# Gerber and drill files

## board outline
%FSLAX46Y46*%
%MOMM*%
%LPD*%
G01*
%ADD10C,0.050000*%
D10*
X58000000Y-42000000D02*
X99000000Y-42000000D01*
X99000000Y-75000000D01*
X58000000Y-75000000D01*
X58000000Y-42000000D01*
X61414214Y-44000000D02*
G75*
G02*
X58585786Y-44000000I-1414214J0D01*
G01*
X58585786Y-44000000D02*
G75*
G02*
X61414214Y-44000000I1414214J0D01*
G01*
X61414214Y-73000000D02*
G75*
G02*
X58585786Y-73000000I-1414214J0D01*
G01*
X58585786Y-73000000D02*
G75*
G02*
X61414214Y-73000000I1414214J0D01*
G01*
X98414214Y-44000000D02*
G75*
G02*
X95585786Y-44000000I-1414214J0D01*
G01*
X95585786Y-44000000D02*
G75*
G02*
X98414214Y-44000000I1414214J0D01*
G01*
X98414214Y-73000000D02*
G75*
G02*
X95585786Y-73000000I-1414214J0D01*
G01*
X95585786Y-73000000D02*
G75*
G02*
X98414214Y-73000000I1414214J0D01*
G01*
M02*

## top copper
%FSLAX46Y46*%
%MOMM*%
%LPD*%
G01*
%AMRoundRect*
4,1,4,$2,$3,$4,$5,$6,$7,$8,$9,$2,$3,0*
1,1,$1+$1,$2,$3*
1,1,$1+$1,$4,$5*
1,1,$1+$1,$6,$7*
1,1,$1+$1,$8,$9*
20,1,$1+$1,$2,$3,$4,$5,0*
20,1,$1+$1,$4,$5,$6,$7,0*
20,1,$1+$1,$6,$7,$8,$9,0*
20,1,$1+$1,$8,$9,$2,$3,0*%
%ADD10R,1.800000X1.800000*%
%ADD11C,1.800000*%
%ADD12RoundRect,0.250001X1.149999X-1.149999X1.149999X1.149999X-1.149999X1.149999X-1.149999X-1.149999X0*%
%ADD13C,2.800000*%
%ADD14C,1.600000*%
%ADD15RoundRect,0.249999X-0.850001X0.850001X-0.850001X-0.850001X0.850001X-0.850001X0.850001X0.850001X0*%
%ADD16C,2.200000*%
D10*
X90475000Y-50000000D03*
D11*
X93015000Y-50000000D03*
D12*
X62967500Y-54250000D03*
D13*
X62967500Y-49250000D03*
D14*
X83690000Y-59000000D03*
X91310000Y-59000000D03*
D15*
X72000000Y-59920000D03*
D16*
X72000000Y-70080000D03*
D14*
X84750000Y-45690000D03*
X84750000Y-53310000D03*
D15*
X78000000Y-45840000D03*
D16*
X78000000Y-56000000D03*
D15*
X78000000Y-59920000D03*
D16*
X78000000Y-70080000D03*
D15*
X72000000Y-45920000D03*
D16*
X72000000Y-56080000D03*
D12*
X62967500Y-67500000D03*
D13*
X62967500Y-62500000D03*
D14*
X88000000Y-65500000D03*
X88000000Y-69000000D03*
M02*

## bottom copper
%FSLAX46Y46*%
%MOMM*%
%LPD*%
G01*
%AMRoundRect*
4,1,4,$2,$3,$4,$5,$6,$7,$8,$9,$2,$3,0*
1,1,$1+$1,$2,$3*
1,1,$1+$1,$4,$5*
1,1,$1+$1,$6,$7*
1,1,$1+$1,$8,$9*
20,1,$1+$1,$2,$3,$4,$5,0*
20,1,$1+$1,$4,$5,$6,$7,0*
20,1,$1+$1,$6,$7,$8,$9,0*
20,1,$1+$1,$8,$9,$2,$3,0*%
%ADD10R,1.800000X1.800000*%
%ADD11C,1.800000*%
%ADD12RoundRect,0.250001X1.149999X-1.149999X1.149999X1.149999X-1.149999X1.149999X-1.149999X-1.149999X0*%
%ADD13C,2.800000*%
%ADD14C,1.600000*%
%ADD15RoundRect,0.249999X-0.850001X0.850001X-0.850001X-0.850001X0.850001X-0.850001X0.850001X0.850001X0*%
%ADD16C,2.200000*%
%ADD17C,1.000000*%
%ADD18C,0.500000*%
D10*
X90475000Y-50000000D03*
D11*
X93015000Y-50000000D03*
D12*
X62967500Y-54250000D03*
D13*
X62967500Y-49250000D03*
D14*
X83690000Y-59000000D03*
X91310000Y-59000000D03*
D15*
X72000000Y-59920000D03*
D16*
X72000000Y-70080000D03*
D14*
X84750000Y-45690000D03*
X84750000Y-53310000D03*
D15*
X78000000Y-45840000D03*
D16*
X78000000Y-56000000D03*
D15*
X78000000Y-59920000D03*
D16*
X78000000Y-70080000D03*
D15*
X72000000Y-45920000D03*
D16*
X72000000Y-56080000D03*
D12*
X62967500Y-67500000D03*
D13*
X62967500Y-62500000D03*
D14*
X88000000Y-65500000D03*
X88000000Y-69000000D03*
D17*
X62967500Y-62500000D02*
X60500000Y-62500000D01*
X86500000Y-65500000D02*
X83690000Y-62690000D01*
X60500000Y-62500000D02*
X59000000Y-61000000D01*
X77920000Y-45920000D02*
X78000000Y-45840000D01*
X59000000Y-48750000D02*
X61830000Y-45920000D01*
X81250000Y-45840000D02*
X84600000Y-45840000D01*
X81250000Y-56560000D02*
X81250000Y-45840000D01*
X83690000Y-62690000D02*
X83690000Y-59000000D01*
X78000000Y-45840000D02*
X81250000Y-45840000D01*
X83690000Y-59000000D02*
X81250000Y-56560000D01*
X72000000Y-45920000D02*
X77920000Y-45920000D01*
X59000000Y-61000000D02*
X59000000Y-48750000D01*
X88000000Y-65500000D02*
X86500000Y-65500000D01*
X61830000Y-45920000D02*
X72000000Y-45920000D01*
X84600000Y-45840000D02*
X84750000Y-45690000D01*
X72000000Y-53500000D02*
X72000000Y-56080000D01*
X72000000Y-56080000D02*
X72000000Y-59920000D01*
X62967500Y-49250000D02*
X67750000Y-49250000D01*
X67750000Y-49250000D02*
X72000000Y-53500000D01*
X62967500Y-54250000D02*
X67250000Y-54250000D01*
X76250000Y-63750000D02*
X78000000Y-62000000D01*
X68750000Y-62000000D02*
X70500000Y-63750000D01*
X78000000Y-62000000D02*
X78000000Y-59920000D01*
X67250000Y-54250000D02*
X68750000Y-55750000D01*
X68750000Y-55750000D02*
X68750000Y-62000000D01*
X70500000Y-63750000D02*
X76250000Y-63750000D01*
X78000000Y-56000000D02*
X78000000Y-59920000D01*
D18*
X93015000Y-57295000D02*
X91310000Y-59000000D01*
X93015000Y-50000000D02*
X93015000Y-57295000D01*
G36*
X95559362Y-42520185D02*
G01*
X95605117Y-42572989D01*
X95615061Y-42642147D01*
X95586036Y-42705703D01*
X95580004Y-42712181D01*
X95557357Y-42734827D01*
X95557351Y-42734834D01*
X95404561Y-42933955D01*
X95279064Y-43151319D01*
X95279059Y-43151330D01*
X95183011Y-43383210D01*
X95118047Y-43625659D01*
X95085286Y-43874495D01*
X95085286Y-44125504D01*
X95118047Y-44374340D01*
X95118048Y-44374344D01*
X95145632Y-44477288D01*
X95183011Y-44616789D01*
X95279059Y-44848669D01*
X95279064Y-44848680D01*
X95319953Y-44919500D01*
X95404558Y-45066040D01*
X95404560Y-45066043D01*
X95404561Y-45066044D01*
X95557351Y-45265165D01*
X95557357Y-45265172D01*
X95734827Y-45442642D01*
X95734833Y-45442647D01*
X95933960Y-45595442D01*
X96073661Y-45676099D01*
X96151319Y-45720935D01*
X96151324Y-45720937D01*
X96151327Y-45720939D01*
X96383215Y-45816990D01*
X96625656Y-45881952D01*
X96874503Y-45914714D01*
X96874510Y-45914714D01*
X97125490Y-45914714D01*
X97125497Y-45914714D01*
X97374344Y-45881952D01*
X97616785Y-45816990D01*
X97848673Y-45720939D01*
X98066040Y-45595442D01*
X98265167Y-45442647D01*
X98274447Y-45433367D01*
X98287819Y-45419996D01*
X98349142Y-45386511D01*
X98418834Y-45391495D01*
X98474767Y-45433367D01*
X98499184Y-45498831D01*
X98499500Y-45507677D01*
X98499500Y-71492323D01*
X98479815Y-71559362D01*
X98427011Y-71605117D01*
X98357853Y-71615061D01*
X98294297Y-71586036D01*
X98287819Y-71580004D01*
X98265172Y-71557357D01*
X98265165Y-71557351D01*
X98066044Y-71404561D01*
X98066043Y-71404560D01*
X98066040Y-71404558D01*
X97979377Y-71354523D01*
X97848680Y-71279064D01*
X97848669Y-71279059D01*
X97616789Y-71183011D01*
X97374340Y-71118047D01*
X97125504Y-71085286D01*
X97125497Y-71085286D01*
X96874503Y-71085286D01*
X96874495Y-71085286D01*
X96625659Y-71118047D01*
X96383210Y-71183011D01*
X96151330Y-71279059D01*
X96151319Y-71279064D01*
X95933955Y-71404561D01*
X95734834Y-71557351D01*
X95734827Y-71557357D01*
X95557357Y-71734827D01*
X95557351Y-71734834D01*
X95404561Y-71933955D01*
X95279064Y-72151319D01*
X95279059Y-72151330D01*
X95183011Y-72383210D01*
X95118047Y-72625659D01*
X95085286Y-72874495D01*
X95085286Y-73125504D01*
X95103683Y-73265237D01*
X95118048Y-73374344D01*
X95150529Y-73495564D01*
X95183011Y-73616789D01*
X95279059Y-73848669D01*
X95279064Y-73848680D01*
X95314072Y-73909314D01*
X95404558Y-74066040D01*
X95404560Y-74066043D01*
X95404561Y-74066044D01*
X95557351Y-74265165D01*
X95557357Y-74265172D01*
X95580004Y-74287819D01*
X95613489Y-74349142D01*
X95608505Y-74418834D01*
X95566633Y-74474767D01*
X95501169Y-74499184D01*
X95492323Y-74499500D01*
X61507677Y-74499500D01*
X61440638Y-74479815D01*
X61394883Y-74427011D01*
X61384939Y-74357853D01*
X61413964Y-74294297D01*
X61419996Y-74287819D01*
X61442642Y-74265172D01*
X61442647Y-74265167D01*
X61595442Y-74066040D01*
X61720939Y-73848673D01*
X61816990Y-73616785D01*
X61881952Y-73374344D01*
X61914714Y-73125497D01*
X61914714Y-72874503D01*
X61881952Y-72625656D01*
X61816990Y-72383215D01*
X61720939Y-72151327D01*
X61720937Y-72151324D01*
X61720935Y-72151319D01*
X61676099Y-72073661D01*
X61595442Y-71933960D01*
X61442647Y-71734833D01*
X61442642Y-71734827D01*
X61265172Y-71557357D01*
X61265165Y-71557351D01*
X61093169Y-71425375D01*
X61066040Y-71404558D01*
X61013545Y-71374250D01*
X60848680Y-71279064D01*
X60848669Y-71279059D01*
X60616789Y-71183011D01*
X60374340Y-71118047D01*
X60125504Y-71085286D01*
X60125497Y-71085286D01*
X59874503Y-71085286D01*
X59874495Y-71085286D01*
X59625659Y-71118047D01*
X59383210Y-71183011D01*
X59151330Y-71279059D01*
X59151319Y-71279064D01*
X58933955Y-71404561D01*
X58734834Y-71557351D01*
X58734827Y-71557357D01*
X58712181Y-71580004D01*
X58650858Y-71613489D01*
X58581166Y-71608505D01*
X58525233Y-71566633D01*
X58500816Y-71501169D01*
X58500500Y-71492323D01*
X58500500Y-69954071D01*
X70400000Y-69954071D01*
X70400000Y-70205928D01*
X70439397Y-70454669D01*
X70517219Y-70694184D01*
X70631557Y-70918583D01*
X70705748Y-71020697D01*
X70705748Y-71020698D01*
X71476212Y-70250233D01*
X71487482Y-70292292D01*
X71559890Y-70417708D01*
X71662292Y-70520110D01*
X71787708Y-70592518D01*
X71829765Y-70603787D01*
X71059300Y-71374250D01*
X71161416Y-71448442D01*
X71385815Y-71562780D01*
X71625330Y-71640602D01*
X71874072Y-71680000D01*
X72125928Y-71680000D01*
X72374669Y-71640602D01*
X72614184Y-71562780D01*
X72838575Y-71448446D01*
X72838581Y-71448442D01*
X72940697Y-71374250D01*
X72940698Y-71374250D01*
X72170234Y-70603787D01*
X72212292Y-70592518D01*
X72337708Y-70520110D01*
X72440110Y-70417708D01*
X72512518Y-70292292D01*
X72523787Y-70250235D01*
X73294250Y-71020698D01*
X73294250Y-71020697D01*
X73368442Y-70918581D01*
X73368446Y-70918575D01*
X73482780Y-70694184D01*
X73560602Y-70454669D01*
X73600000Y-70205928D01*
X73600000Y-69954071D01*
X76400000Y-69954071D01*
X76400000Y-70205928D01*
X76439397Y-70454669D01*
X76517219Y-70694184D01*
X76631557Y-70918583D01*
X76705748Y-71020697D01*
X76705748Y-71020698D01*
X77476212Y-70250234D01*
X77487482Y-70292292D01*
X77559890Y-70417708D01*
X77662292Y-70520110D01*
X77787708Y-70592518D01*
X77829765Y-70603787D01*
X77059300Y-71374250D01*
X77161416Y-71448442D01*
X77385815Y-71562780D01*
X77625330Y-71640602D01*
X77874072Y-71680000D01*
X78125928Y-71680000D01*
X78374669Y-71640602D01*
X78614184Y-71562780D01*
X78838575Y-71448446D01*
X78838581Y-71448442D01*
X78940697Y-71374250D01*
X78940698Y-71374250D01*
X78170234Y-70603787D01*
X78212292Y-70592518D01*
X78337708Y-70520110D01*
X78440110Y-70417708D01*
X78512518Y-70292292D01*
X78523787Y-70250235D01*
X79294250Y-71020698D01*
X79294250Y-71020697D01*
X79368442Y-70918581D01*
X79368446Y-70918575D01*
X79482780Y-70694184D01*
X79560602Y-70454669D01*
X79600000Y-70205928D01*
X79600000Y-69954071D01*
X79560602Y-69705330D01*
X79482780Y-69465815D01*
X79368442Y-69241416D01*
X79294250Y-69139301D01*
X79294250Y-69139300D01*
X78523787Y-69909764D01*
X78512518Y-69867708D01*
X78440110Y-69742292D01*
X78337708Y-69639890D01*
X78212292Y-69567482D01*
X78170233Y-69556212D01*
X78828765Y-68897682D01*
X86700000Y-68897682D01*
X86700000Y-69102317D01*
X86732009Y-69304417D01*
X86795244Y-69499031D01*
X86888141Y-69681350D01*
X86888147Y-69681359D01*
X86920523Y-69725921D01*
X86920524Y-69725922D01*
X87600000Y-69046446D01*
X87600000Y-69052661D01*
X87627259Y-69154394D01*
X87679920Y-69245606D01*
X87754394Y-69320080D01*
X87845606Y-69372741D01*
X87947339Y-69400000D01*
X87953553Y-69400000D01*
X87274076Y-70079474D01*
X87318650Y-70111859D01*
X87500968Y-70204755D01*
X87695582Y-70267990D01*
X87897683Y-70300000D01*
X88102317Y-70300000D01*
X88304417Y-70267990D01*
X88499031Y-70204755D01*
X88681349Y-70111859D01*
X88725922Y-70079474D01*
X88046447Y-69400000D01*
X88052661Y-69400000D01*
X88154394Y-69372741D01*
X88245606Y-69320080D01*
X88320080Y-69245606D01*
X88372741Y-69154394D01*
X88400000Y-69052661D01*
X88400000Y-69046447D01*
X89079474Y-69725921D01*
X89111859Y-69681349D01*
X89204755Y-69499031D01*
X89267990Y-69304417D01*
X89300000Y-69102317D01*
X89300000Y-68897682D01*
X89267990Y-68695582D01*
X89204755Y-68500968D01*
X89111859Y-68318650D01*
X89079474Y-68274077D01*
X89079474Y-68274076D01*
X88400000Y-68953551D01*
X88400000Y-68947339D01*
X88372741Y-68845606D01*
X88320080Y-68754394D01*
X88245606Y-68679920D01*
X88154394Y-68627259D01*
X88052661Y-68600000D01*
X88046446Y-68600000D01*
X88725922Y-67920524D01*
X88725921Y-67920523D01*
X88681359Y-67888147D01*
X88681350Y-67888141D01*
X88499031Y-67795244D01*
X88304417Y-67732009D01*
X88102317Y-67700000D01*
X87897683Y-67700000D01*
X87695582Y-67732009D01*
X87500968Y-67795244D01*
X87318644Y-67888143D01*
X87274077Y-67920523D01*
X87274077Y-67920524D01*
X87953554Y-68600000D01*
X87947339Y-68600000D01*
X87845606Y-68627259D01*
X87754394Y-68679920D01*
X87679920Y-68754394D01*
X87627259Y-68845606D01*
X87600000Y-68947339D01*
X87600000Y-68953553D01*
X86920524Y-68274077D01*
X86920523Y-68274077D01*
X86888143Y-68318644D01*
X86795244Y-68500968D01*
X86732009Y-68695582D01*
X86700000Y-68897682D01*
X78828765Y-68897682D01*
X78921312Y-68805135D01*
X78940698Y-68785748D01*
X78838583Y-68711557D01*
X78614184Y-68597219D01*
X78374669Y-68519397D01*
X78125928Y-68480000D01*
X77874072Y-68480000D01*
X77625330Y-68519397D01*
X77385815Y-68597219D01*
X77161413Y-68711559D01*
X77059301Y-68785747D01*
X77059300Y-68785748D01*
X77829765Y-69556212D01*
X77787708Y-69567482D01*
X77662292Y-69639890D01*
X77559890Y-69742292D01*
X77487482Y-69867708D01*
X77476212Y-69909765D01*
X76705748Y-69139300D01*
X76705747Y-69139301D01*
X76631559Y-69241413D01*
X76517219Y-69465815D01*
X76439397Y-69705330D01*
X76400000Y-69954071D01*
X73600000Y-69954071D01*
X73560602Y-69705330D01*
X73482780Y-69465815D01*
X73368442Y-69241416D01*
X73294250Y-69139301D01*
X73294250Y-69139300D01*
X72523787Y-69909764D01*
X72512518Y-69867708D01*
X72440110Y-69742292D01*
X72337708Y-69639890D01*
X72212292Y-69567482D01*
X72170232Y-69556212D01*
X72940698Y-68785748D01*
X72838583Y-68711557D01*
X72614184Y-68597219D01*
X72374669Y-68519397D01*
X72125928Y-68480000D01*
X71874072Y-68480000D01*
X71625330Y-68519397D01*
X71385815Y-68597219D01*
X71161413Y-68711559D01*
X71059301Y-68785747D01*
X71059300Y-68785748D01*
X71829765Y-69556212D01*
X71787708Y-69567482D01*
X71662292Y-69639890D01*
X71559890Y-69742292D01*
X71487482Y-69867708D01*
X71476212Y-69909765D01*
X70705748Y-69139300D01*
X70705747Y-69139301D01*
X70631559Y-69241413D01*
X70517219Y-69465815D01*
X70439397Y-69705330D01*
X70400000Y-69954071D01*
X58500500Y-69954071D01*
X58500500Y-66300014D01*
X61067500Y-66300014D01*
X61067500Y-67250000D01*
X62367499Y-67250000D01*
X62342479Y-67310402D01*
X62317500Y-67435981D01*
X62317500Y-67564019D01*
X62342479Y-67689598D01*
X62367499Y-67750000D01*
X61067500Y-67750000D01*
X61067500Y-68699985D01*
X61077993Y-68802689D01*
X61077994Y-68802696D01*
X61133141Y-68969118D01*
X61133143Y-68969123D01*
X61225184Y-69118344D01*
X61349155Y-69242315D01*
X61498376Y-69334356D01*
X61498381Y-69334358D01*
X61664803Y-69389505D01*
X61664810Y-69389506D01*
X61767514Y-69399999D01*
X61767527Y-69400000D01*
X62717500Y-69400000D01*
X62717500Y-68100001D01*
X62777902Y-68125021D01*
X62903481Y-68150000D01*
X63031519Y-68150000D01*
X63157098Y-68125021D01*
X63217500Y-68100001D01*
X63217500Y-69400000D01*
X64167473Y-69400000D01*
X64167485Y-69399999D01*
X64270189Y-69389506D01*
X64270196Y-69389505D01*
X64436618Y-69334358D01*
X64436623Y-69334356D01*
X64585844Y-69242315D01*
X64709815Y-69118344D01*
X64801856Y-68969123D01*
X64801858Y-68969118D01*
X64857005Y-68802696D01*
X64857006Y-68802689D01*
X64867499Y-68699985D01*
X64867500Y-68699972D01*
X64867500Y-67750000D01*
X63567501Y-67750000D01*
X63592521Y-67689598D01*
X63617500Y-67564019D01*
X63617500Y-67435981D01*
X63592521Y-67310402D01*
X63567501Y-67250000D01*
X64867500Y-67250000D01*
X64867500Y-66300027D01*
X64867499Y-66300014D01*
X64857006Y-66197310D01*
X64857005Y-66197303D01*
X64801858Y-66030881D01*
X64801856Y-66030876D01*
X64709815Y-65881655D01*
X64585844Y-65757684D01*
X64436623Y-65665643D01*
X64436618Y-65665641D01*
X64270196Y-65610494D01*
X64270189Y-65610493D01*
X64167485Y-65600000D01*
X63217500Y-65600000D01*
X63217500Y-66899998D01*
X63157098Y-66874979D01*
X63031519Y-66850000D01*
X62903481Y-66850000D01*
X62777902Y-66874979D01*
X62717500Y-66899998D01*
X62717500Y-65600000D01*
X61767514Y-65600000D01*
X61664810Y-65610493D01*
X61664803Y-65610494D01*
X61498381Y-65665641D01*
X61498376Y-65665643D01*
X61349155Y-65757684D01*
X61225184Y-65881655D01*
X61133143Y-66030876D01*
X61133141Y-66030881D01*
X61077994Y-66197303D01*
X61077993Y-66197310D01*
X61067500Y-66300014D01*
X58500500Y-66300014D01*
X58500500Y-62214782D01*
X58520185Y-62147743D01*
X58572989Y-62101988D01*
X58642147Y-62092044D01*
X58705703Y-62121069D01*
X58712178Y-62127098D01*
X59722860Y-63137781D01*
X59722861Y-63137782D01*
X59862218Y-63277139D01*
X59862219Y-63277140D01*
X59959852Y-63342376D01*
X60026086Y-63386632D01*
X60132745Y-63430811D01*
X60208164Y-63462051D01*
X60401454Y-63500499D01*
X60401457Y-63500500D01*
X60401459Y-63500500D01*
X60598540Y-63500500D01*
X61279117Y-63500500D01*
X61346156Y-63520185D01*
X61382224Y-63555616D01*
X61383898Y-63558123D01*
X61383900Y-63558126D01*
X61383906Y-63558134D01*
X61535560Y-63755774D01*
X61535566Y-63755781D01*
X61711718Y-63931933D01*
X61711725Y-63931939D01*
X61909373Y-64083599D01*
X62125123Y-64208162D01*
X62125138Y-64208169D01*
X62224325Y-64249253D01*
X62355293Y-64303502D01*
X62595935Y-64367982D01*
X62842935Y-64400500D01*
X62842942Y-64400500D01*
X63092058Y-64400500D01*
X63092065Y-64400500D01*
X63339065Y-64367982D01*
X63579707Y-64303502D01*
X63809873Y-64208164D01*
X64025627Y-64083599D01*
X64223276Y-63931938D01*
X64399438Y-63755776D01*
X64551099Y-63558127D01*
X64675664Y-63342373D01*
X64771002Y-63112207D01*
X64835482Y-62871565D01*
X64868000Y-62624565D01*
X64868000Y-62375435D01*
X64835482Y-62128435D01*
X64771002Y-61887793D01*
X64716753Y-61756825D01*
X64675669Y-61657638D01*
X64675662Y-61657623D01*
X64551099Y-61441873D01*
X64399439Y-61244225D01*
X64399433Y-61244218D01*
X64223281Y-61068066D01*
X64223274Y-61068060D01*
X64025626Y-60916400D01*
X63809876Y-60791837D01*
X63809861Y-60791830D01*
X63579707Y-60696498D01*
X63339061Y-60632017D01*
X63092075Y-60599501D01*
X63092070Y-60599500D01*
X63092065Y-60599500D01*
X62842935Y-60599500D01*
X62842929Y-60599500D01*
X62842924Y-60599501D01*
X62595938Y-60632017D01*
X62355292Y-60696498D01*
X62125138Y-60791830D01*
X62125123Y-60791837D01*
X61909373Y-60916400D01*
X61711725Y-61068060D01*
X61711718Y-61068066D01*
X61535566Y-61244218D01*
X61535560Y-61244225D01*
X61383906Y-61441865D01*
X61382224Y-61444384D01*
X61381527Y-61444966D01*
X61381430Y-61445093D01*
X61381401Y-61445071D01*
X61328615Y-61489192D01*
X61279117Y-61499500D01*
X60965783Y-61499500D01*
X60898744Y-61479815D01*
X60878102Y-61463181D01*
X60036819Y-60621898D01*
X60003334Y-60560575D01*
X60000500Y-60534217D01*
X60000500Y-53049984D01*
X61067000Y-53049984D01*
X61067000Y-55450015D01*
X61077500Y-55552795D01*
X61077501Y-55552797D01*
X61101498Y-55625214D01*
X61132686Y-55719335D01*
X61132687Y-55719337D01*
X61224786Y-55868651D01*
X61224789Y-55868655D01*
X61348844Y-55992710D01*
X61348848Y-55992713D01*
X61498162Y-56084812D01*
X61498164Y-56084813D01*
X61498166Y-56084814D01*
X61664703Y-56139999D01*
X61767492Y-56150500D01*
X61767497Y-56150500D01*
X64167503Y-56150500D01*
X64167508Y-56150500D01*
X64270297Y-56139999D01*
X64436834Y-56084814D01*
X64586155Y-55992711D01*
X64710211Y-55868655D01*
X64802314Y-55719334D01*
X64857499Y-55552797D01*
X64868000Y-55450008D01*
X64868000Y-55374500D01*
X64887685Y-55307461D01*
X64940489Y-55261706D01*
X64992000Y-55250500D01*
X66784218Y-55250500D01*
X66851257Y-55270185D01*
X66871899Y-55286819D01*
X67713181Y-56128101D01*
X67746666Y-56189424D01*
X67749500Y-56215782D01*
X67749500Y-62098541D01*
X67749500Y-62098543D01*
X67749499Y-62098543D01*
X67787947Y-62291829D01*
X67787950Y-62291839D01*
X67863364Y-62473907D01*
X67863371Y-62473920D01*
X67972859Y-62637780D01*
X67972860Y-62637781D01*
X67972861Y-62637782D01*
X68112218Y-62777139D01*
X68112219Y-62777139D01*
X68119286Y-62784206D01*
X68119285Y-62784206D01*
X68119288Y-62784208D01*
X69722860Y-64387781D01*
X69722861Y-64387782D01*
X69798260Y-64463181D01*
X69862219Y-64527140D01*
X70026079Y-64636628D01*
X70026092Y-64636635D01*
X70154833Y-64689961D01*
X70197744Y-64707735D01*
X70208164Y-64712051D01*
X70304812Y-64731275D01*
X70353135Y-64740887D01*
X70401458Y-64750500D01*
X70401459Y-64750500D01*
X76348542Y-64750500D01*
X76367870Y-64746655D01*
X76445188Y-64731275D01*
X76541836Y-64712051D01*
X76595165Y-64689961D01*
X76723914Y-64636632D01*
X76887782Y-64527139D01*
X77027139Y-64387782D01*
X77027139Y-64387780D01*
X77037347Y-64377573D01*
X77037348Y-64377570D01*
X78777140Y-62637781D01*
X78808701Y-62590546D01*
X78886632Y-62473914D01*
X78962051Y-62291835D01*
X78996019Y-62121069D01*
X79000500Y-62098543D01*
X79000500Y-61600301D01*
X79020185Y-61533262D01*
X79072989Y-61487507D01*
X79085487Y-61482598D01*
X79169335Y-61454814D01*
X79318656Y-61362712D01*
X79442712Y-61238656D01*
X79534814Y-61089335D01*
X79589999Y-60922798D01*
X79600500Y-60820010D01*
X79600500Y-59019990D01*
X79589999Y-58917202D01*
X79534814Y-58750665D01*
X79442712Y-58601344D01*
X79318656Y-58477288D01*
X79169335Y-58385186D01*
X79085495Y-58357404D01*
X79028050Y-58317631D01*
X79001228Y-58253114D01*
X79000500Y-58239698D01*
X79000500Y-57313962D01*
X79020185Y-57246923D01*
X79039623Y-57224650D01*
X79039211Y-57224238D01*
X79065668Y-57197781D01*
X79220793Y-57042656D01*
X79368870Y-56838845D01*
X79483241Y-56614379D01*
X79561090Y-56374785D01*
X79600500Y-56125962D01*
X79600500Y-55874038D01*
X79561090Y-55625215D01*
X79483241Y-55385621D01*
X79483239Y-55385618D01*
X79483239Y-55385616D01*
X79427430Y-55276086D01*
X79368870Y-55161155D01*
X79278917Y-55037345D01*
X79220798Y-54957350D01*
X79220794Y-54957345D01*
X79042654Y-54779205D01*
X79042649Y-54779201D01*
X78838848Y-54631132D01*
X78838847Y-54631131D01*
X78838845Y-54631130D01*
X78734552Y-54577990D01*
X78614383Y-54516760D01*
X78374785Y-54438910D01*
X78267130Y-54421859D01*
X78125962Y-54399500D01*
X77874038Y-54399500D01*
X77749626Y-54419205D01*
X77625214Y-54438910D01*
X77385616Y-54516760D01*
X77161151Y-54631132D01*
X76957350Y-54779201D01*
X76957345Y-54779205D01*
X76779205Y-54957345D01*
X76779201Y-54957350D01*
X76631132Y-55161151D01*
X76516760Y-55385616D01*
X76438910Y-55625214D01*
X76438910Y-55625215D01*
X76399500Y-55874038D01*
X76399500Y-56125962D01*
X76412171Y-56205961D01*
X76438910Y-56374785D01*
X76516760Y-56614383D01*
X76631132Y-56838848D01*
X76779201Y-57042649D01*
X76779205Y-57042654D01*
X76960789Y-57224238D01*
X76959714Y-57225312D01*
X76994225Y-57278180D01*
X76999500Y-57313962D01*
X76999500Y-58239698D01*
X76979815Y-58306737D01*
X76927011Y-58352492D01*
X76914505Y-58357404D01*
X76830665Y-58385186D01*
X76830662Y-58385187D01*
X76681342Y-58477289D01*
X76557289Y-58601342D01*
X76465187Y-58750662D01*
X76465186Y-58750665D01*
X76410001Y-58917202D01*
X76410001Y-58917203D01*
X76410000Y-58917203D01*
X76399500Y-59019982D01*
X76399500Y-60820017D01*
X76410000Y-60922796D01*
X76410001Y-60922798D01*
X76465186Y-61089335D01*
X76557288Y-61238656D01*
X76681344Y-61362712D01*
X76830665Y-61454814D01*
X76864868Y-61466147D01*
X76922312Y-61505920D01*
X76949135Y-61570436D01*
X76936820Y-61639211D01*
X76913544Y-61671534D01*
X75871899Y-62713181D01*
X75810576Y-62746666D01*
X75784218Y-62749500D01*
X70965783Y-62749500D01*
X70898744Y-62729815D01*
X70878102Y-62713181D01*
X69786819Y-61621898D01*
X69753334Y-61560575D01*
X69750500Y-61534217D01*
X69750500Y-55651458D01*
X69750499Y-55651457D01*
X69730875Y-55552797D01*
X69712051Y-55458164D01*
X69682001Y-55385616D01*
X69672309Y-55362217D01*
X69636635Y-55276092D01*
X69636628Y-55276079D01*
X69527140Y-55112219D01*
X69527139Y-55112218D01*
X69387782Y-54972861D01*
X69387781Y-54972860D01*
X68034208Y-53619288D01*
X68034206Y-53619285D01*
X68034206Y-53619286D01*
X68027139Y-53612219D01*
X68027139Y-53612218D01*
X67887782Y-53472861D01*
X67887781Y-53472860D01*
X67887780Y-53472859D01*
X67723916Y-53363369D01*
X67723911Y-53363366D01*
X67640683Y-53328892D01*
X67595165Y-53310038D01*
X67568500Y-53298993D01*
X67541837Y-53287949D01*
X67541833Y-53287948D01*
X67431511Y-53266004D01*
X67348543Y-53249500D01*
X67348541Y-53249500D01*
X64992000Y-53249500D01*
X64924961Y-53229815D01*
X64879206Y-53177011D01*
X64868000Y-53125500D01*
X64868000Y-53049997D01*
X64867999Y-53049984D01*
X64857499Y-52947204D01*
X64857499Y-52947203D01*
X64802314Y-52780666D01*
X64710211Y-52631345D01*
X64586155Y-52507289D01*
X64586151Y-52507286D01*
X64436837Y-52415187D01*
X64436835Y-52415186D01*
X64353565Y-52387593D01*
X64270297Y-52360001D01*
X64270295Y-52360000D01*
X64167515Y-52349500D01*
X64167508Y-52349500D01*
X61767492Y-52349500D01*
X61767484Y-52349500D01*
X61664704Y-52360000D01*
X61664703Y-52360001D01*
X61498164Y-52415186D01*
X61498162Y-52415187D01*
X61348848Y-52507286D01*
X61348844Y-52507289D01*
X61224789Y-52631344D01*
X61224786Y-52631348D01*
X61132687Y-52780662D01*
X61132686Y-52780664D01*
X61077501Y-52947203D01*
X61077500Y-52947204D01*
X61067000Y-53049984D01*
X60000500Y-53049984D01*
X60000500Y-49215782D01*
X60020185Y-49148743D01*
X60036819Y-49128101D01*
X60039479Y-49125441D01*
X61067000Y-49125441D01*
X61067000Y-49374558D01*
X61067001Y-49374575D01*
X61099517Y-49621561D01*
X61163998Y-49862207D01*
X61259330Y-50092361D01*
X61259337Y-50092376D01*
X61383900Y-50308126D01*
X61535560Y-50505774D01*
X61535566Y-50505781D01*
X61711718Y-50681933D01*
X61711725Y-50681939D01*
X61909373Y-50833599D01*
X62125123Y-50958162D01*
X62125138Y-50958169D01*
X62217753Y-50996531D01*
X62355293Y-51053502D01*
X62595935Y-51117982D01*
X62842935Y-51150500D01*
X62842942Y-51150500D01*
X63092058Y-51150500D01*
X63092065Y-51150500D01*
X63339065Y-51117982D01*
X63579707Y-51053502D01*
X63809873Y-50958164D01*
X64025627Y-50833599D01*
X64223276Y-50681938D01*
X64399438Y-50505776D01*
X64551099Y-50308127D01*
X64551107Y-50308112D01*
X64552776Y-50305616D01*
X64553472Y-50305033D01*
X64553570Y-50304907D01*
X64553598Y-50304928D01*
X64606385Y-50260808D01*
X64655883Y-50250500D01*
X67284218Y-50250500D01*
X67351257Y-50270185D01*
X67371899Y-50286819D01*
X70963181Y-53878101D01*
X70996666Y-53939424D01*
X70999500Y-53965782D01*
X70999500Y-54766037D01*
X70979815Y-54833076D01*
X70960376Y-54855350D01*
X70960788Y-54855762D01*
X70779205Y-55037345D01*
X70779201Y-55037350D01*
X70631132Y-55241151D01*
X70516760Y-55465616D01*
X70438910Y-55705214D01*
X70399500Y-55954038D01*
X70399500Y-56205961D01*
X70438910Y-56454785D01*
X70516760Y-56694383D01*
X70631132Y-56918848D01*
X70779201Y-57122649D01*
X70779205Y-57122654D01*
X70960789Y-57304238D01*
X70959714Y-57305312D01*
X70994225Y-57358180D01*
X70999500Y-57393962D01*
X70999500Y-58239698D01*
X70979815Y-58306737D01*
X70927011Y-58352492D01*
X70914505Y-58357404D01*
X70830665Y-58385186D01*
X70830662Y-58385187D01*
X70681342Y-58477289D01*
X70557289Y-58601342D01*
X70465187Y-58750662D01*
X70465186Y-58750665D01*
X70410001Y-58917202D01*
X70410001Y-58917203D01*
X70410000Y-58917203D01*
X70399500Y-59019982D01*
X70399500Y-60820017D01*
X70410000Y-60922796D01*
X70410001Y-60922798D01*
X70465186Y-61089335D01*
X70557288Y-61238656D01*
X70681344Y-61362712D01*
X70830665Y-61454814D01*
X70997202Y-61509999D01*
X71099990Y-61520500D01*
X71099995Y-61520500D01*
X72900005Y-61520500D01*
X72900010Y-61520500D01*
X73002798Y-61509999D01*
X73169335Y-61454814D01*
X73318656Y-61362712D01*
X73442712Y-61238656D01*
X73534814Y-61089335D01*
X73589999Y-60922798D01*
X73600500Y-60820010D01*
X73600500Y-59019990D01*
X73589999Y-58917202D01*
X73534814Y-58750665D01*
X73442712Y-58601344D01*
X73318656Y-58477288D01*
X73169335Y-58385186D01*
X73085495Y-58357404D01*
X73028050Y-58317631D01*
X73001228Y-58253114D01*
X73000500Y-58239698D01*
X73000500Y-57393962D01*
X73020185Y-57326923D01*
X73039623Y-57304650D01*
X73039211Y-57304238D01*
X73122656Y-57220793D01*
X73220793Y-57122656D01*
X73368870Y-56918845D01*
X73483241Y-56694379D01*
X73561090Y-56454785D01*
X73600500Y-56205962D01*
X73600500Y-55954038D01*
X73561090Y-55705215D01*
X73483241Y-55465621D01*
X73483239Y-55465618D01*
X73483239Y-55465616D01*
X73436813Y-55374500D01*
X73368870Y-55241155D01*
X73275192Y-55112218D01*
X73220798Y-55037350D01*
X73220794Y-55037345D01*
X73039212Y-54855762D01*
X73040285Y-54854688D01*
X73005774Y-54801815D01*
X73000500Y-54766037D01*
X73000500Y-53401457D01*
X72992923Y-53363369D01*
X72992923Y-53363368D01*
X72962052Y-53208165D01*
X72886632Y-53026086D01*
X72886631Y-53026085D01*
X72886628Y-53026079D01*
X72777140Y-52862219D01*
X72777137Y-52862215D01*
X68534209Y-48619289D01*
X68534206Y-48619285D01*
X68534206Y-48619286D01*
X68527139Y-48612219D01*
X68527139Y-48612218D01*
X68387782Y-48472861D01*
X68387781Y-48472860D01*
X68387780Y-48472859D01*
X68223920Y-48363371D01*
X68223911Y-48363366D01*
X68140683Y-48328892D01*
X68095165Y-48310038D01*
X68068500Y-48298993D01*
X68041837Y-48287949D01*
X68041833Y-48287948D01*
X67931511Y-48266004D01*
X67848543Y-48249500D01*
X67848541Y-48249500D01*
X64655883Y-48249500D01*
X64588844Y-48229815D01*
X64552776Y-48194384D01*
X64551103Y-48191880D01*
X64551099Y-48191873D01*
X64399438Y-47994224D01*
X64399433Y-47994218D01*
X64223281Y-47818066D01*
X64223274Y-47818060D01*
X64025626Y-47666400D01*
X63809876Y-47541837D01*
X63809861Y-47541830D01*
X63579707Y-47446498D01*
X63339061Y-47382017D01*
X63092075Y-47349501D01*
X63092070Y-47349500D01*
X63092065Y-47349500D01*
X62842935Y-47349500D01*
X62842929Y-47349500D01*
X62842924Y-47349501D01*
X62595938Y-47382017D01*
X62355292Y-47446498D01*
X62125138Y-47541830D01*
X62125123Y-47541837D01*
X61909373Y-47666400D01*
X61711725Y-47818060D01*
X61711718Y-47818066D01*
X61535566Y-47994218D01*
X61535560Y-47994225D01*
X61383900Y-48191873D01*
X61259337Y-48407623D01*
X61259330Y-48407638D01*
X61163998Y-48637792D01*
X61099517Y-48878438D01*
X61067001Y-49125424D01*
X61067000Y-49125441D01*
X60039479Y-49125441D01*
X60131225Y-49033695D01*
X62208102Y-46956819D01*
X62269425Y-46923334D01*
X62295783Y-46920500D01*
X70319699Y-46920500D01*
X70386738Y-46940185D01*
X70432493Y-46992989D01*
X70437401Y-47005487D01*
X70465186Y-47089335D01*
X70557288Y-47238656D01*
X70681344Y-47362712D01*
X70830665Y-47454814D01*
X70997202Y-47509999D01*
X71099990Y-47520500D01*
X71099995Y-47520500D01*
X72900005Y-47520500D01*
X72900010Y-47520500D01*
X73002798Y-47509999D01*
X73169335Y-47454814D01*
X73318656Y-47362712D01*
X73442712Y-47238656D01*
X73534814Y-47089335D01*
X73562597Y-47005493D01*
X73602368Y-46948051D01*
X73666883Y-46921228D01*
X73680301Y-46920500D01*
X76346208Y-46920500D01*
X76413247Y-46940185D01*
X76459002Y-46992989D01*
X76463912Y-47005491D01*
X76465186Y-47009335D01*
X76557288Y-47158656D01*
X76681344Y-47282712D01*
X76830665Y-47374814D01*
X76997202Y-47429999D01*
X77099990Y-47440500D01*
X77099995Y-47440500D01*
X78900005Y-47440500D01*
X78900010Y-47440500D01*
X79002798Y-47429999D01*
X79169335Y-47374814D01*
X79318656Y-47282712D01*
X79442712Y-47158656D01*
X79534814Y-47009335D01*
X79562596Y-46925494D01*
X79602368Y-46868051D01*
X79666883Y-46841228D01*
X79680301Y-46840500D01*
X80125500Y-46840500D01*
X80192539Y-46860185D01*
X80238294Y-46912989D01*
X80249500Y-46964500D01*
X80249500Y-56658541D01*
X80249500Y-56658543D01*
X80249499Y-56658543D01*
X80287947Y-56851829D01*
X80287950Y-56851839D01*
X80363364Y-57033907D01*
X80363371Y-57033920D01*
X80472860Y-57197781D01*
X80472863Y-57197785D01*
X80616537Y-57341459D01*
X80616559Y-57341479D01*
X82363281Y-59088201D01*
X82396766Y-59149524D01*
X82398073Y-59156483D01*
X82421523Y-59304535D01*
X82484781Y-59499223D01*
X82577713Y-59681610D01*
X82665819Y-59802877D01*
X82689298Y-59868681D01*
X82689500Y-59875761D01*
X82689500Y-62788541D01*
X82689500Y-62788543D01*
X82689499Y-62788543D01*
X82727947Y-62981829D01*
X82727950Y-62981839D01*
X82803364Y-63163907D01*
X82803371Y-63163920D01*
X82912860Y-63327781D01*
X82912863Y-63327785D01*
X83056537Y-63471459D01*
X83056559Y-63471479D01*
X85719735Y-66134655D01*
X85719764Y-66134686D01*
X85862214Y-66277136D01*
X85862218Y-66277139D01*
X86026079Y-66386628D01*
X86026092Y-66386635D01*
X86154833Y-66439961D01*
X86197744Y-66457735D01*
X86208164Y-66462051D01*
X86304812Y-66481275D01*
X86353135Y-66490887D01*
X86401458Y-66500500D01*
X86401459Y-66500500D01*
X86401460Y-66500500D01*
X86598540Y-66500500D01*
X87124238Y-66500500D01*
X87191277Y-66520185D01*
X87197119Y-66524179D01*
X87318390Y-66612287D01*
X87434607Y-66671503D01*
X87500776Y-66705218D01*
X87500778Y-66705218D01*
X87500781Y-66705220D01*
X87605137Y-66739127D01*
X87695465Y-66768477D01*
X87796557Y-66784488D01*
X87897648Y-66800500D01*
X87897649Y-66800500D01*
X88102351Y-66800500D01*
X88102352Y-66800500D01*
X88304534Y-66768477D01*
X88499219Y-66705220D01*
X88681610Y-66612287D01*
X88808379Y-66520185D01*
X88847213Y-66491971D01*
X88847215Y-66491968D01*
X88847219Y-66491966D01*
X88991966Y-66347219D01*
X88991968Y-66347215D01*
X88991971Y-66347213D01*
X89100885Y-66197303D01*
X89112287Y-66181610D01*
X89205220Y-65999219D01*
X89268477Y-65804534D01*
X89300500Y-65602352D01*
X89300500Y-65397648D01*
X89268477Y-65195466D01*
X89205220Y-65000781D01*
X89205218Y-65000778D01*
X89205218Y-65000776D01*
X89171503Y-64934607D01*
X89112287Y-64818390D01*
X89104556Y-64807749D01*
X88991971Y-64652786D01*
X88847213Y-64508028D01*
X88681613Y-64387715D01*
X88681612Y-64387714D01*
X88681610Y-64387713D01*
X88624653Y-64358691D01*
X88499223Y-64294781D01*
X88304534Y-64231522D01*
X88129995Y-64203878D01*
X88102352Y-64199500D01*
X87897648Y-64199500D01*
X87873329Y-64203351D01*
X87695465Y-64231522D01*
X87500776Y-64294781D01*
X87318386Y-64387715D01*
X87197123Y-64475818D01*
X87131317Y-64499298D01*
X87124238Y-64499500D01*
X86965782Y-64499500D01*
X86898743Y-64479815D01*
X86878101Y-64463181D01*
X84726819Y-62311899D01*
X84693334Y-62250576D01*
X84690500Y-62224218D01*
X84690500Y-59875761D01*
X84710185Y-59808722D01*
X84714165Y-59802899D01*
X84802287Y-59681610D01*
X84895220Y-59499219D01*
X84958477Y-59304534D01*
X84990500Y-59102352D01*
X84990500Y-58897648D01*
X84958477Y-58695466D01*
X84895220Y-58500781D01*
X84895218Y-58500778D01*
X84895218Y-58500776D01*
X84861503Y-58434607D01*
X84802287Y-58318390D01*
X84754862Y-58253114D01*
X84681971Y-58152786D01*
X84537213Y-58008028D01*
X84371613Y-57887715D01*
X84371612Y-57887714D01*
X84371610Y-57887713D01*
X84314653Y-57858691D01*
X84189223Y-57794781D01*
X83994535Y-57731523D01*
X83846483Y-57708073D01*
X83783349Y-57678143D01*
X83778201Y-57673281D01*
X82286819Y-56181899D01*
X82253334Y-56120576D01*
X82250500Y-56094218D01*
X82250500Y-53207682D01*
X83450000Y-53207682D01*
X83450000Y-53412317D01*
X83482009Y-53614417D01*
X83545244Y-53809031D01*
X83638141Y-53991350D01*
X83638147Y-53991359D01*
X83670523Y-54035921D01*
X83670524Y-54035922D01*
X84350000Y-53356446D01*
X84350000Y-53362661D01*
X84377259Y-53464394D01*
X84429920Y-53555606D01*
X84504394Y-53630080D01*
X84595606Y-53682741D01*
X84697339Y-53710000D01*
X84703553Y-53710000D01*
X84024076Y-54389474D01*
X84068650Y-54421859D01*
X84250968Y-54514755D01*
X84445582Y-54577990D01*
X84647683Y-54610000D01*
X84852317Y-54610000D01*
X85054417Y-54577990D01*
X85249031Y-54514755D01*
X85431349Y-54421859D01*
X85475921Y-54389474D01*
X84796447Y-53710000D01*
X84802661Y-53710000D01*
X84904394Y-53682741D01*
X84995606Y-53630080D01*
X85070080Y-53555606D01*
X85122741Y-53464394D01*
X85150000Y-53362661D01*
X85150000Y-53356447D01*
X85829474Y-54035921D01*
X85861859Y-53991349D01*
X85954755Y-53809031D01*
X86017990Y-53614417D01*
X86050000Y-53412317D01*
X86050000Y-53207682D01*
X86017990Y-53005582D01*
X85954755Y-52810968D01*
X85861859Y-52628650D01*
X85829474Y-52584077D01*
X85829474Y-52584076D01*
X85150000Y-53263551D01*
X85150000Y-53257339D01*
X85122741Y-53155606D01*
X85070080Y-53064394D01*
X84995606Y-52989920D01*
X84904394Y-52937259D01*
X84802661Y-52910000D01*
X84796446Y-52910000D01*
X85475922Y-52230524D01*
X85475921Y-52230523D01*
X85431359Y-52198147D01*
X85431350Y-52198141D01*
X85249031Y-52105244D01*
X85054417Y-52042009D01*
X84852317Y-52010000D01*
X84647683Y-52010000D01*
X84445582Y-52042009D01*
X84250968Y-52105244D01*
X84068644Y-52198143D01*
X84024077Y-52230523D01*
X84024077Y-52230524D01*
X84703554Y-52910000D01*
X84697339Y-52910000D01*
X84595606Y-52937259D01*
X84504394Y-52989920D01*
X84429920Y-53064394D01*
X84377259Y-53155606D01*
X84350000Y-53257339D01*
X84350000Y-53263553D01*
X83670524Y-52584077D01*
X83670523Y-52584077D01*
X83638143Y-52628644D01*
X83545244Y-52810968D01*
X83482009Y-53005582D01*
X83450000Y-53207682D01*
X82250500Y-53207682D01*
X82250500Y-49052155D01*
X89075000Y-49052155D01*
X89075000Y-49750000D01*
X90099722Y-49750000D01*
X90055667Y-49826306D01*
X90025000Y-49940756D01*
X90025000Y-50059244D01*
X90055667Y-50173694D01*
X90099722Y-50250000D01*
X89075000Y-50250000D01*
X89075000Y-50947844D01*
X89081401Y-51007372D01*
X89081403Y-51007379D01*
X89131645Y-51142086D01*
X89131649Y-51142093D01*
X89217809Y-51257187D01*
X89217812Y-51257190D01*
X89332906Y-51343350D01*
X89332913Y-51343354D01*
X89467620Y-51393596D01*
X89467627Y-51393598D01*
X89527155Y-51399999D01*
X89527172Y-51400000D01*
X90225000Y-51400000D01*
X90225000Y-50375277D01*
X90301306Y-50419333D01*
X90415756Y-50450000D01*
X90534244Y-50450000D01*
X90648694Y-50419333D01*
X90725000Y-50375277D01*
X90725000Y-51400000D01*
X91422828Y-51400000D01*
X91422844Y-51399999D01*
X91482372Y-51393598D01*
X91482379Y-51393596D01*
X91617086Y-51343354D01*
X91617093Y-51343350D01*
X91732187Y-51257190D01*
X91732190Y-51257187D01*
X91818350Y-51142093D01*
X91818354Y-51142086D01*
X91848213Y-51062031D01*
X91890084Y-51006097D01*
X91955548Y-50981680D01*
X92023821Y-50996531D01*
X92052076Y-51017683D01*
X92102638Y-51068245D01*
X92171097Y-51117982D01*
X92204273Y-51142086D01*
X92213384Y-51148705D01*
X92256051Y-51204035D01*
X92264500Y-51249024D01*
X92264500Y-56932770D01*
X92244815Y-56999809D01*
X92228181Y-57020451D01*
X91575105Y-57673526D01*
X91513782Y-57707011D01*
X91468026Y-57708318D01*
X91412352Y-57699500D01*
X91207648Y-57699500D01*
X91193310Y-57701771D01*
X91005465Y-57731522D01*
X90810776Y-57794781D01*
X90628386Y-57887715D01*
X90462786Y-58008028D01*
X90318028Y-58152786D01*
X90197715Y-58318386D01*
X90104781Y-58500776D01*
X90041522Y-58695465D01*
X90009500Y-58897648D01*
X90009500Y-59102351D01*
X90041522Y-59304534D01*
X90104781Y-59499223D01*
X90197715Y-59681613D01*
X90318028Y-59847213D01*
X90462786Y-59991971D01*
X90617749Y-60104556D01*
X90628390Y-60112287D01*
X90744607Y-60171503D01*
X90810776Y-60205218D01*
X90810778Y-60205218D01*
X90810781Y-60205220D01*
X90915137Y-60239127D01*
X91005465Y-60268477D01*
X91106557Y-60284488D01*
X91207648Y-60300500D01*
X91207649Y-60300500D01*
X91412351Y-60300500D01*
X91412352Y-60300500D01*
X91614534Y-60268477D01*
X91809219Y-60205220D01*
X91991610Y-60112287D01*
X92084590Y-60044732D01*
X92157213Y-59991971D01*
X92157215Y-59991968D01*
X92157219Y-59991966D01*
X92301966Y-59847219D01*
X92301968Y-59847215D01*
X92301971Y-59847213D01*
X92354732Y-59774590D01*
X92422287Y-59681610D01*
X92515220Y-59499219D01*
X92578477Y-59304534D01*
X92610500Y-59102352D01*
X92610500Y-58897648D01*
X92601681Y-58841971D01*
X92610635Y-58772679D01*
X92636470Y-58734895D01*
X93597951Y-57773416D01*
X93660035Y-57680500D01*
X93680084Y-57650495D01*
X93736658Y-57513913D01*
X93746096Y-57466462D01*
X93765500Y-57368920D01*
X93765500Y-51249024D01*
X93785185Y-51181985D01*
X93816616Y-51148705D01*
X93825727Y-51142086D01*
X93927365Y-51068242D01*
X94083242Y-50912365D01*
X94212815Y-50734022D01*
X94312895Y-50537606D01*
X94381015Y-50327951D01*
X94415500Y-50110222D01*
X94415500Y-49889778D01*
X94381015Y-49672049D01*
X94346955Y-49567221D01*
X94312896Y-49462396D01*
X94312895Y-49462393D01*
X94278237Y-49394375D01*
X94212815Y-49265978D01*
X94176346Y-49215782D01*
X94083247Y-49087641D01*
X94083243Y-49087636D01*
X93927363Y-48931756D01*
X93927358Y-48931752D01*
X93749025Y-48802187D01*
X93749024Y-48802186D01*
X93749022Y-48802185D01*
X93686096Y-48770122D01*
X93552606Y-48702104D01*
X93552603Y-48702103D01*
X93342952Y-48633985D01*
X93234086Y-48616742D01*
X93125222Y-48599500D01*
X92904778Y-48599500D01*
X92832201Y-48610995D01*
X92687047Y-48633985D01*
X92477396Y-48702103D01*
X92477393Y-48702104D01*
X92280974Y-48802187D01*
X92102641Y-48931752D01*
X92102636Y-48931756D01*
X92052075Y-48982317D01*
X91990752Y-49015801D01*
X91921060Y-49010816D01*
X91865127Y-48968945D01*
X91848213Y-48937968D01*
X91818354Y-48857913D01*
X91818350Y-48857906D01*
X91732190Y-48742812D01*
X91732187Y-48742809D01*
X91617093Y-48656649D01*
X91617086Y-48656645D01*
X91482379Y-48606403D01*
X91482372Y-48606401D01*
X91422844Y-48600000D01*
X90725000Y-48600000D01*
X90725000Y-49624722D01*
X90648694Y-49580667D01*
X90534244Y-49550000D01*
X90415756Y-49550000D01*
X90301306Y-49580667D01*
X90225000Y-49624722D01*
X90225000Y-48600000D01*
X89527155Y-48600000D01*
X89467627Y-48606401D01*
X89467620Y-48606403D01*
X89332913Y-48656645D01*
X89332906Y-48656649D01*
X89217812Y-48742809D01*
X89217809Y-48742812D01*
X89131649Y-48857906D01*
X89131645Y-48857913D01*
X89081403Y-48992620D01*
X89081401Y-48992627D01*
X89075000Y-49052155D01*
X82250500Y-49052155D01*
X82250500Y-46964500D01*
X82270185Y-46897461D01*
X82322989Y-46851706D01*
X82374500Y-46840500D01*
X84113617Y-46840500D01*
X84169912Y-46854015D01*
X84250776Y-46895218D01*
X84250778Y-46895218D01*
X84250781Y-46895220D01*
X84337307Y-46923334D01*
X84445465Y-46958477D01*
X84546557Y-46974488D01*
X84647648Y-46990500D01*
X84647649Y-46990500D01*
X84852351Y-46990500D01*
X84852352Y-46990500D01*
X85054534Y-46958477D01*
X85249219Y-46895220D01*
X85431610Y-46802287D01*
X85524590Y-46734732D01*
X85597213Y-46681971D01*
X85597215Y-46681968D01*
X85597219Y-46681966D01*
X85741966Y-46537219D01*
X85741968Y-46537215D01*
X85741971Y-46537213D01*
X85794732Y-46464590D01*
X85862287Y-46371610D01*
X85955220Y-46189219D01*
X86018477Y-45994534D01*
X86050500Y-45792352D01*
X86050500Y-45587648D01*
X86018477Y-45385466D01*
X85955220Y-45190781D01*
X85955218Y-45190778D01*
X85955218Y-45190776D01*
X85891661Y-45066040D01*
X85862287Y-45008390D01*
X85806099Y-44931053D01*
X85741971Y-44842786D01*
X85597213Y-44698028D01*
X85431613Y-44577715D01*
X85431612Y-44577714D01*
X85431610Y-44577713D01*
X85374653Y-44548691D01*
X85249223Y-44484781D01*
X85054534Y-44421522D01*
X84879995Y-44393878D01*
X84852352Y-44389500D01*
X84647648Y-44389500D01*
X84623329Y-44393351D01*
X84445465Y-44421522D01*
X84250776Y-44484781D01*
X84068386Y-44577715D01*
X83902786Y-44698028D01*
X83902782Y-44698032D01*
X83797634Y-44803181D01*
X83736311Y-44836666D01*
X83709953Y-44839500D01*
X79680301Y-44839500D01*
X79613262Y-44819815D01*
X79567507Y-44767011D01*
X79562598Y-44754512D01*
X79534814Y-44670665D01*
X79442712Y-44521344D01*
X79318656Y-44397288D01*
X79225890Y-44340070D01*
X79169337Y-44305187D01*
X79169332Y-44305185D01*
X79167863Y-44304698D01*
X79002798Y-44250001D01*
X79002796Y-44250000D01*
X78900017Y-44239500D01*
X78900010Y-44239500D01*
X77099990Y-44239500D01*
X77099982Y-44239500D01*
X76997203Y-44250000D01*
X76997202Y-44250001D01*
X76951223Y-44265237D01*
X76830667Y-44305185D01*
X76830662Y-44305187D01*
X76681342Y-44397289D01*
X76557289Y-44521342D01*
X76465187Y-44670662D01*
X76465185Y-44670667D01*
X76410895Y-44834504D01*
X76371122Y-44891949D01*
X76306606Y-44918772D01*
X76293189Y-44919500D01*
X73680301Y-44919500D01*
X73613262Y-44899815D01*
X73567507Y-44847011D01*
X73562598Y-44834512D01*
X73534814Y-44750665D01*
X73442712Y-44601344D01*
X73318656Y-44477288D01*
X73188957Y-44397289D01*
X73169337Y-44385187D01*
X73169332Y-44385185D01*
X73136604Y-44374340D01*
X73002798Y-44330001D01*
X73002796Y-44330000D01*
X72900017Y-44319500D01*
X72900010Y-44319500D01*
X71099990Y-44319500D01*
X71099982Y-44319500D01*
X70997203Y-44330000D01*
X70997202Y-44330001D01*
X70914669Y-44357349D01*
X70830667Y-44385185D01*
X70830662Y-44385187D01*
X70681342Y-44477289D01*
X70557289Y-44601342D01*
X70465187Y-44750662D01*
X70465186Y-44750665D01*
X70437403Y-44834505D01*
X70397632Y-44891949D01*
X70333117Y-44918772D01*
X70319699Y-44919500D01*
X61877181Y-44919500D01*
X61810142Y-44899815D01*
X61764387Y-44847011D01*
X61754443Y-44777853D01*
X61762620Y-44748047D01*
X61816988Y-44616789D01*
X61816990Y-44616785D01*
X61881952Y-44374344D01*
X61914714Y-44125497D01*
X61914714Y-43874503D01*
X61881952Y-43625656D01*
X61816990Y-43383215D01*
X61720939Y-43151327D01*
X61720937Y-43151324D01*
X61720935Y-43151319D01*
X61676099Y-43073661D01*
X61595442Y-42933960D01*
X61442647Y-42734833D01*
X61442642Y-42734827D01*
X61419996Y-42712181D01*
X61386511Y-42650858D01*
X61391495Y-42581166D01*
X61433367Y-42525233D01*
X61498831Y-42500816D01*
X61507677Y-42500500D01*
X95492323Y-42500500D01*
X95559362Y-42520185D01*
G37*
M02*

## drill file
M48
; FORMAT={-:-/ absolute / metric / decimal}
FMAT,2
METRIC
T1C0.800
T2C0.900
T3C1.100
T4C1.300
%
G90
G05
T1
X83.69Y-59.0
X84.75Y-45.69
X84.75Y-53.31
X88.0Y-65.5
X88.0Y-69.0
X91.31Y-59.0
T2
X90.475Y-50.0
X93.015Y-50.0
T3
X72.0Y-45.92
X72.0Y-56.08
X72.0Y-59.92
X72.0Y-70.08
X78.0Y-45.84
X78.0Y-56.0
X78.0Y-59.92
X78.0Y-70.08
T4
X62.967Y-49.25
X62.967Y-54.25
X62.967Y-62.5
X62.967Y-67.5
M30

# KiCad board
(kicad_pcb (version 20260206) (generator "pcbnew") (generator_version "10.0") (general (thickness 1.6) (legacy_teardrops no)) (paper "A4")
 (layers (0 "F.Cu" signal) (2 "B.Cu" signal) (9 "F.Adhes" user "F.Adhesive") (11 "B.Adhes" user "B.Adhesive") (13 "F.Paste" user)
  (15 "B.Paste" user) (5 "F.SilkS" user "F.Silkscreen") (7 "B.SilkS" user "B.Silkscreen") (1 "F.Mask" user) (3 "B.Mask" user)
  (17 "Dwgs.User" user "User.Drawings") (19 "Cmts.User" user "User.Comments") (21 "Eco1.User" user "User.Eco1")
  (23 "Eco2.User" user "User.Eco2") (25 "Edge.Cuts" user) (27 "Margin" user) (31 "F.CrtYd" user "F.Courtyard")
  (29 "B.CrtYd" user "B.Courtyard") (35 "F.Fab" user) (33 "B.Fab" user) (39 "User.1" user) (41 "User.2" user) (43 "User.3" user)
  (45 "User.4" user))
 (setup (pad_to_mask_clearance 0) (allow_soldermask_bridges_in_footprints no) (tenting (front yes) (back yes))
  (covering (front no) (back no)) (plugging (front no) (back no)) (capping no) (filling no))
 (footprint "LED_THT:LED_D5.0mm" (layer "F.Cu") (at 90.475 50)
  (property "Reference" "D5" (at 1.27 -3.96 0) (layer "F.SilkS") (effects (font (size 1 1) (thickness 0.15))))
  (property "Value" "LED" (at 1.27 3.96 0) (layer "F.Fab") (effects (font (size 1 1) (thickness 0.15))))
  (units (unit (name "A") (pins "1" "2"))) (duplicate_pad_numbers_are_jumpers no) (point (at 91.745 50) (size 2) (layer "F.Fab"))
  (pad "1" thru_hole rect (at 0 0) (size 1.8 1.8) (drill 0.9) (layers "*.Cu" "*.Mask") (remove_unused_layers no) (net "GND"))
  (pad "2" thru_hole circle (at 2.54 0) (size 1.8 1.8) (drill 0.9) (layers "*.Cu" "*.Mask") (remove_unused_layers no) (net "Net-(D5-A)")))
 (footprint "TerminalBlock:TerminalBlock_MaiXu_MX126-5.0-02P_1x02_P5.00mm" (layer "F.Cu") (at 62.9675 54.25 90)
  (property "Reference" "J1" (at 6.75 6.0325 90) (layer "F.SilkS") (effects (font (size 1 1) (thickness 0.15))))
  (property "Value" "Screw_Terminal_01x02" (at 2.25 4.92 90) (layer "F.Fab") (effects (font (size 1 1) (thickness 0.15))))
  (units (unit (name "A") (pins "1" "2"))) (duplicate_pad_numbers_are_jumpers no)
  (pad "1" thru_hole roundrect (at 0 0 90) (size 2.8 2.8) (drill 1.3) (layers "*.Cu" "*.Mask") (remove_unused_layers no)
   (roundrect_rratio 0.089286) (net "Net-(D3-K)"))
  (pad "2" thru_hole circle (at 5 0 90) (size 2.8 2.8) (drill 1.3) (layers "*.Cu" "*.Mask") (remove_unused_layers no) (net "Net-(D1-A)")))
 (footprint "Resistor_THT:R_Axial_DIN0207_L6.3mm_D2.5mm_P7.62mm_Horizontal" (layer "F.Cu") (at 83.69 59)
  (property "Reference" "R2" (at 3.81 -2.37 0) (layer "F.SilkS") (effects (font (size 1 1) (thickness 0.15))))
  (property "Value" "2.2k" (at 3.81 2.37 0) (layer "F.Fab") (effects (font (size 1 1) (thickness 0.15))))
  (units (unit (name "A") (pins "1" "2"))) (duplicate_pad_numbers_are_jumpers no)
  (pad "1" thru_hole circle (at 0 0) (size 1.6 1.6) (drill 0.8) (layers "*.Cu" "*.Mask") (remove_unused_layers no) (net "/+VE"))
  (pad "2" thru_hole circle (at 7.62 0) (size 1.6 1.6) (drill 0.8) (layers "*.Cu" "*.Mask") (remove_unused_layers no) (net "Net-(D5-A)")))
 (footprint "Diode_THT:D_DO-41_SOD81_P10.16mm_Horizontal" (layer "F.Cu") (at 72 59.92 -90)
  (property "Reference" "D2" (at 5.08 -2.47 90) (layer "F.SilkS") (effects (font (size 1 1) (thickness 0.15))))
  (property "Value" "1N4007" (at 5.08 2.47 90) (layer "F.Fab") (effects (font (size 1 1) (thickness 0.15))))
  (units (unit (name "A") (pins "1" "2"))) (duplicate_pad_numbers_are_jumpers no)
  (pad "1" thru_hole roundrect (at 0 0 270) (size 2.2 2.2) (drill 1.1) (layers "*.Cu" "*.Mask") (remove_unused_layers no)
   (roundrect_rratio 0.113636) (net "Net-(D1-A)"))
  (pad "2" thru_hole circle (at 10.16 0 270) (size 2.2 2.2) (drill 1.1) (layers "*.Cu" "*.Mask") (remove_unused_layers no) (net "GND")))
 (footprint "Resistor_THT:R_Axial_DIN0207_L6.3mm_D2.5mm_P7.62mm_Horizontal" (layer "F.Cu") (at 84.75 45.69 -90)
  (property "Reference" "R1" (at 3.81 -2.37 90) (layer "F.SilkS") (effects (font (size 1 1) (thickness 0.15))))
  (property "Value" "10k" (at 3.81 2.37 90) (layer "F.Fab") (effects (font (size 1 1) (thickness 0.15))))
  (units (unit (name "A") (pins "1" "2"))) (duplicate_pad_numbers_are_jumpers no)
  (pad "1" thru_hole circle (at 0 0 270) (size 1.6 1.6) (drill 0.8) (layers "*.Cu" "*.Mask") (remove_unused_layers no) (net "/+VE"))
  (pad "2" thru_hole circle (at 7.62 0 270) (size 1.6 1.6) (drill 0.8) (layers "*.Cu" "*.Mask") (remove_unused_layers no) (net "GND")))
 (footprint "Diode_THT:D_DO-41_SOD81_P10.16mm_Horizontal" (layer "F.Cu") (at 78 45.84 -90)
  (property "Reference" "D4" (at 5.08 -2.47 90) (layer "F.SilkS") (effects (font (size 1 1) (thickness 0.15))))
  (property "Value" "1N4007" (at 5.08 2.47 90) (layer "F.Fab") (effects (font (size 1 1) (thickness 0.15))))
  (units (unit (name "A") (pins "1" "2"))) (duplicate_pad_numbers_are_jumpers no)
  (pad "1" thru_hole roundrect (at 0 0 270) (size 2.2 2.2) (drill 1.1) (layers "*.Cu" "*.Mask") (remove_unused_layers no)
   (roundrect_rratio 0.113636) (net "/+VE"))
  (pad "2" thru_hole circle (at 10.16 0 270) (size 2.2 2.2) (drill 1.1) (layers "*.Cu" "*.Mask") (remove_unused_layers no)
   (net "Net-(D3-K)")))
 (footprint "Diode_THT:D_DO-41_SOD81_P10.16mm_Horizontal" (layer "F.Cu") (at 78 59.92 -90)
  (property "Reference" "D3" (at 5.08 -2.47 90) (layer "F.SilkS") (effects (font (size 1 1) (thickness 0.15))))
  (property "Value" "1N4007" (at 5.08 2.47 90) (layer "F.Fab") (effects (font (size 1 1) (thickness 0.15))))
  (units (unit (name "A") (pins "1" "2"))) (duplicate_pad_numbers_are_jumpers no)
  (pad "1" thru_hole roundrect (at 0 0 270) (size 2.2 2.2) (drill 1.1) (layers "*.Cu" "*.Mask") (remove_unused_layers no)
   (roundrect_rratio 0.113636) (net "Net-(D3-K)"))
  (pad "2" thru_hole circle (at 10.16 0 270) (size 2.2 2.2) (drill 1.1) (layers "*.Cu" "*.Mask") (remove_unused_layers no) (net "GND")))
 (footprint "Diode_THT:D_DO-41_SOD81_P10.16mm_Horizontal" (layer "F.Cu") (at 72 45.92 -90)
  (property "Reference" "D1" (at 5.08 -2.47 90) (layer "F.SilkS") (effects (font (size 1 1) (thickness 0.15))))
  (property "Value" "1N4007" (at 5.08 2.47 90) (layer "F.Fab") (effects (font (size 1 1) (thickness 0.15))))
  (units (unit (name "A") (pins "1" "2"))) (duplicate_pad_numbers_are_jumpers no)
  (pad "1" thru_hole roundrect (at 0 0 270) (size 2.2 2.2) (drill 1.1) (layers "*.Cu" "*.Mask") (remove_unused_layers no)
   (roundrect_rratio 0.113636) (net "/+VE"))
  (pad "2" thru_hole circle (at 10.16 0 270) (size 2.2 2.2) (drill 1.1) (layers "*.Cu" "*.Mask") (remove_unused_layers no)
   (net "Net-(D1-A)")))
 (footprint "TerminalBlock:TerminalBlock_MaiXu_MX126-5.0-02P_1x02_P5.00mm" (layer "F.Cu") (at 62.9675 67.5 90)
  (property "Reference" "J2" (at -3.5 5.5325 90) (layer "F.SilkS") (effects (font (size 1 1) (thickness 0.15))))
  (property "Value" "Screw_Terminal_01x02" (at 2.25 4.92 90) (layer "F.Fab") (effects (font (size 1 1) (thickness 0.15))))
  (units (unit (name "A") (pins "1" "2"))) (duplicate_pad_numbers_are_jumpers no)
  (pad "1" thru_hole roundrect (at 0 0 90) (size 2.8 2.8) (drill 1.3) (layers "*.Cu" "*.Mask") (remove_unused_layers no)
   (roundrect_rratio 0.089286) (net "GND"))
  (pad "2" thru_hole circle (at 5 0 90) (size 2.8 2.8) (drill 1.3) (layers "*.Cu" "*.Mask") (remove_unused_layers no) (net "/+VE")))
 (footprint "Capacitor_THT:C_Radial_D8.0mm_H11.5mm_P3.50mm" (layer "F.Cu") (at 88 65.5 -90)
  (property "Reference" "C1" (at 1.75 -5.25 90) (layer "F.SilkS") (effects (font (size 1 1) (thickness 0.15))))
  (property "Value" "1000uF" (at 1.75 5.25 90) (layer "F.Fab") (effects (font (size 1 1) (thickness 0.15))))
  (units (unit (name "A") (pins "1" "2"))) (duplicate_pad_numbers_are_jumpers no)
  (pad "1" thru_hole circle (at 0 0 270) (size 1.6 1.6) (drill 0.8) (layers "*.Cu" "*.Mask") (remove_unused_layers no) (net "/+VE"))
  (pad "2" thru_hole circle (at 3.5 0 270) (size 1.6 1.6) (drill 0.8) (layers "*.Cu" "*.Mask") (remove_unused_layers no) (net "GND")))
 (gr_rect (start 58 42) (end 99 75) (stroke (width 0.05) (type default)) (fill no) (layer "Edge.Cuts"))
 (gr_circle (center 60 44) (end 61 45) (stroke (width 0.05) (type default)) (fill no) (layer "Edge.Cuts"))
 (gr_circle (center 60 73) (end 61 74) (stroke (width 0.05) (type default)) (fill no) (layer "Edge.Cuts"))
 (gr_circle (center 97 44) (end 98 45) (stroke (width 0.05) (type default)) (fill no) (layer "Edge.Cuts"))
 (gr_circle (center 97 73) (end 98 74) (stroke (width 0.05) (type default)) (fill no) (layer "Edge.Cuts"))
 (segment (start 62.9675 62.5) (end 60.5 62.5) (width 1) (layer "B.Cu") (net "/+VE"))
 (segment (start 86.5 65.5) (end 83.69 62.69) (width 1) (layer "B.Cu") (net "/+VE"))
 (segment (start 60.5 62.5) (end 59 61) (width 1) (layer "B.Cu") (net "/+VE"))
 (segment (start 77.92 45.92) (end 78 45.84) (width 1) (layer "B.Cu") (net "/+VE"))
 (segment (start 59 48.75) (end 61.83 45.92) (width 1) (layer "B.Cu") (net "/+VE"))
 (segment (start 81.25 45.84) (end 84.6 45.84) (width 1) (layer "B.Cu") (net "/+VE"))
 (segment (start 81.25 56.56) (end 81.25 45.84) (width 1) (layer "B.Cu") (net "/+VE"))
 (segment (start 83.69 62.69) (end 83.69 59) (width 1) (layer "B.Cu") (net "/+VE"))
 (segment (start 78 45.84) (end 81.25 45.84) (width 1) (layer "B.Cu") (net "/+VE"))
 (segment (start 83.69 59) (end 81.25 56.56) (width 1) (layer "B.Cu") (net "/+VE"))
 (segment (start 72 45.92) (end 77.92 45.92) (width 1) (layer "B.Cu") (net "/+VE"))
 (segment (start 59 61) (end 59 48.75) (width 1) (layer "B.Cu") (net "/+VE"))
 (segment (start 88 65.5) (end 86.5 65.5) (width 1) (layer "B.Cu") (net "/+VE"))
 (segment (start 61.83 45.92) (end 72 45.92) (width 1) (layer "B.Cu") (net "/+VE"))
 (segment (start 84.6 45.84) (end 84.75 45.69) (width 1) (layer "B.Cu") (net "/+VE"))
 (segment (start 72 53.5) (end 72 56.08) (width 1) (layer "B.Cu") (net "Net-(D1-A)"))
 (segment (start 72 56.08) (end 72 59.92) (width 1) (layer "B.Cu") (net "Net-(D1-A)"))
 (segment (start 62.9675 49.25) (end 67.75 49.25) (width 1) (layer "B.Cu") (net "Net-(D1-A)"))
 (segment (start 67.75 49.25) (end 72 53.5) (width 1) (layer "B.Cu") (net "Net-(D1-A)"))
 (segment (start 62.9675 54.25) (end 67.25 54.25) (width 1) (layer "B.Cu") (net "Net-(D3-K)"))
 (segment (start 76.25 63.75) (end 78 62) (width 1) (layer "B.Cu") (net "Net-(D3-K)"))
 (segment (start 68.75 62) (end 70.5 63.75) (width 1) (layer "B.Cu") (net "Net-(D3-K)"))
 (segment (start 78 62) (end 78 59.92) (width 1) (layer "B.Cu") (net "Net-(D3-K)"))
 (segment (start 67.25 54.25) (end 68.75 55.75) (width 1) (layer "B.Cu") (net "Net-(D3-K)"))
 (segment (start 68.75 55.75) (end 68.75 62) (width 1) (layer "B.Cu") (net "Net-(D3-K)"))
 (segment (start 70.5 63.75) (end 76.25 63.75) (width 1) (layer "B.Cu") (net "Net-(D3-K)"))
 (segment (start 78 56) (end 78 59.92) (width 1) (layer "B.Cu") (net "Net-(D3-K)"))
 (segment (start 93.015 57.295) (end 91.31 59) (width 0.5) (layer "B.Cu") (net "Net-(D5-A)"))
 (segment (start 93.015 50) (end 93.015 57.295) (width 0.5) (layer "B.Cu") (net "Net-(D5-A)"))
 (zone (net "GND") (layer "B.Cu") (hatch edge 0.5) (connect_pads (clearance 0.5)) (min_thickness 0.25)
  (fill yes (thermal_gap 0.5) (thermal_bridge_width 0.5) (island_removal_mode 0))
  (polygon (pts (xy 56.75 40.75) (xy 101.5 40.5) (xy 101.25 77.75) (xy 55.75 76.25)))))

